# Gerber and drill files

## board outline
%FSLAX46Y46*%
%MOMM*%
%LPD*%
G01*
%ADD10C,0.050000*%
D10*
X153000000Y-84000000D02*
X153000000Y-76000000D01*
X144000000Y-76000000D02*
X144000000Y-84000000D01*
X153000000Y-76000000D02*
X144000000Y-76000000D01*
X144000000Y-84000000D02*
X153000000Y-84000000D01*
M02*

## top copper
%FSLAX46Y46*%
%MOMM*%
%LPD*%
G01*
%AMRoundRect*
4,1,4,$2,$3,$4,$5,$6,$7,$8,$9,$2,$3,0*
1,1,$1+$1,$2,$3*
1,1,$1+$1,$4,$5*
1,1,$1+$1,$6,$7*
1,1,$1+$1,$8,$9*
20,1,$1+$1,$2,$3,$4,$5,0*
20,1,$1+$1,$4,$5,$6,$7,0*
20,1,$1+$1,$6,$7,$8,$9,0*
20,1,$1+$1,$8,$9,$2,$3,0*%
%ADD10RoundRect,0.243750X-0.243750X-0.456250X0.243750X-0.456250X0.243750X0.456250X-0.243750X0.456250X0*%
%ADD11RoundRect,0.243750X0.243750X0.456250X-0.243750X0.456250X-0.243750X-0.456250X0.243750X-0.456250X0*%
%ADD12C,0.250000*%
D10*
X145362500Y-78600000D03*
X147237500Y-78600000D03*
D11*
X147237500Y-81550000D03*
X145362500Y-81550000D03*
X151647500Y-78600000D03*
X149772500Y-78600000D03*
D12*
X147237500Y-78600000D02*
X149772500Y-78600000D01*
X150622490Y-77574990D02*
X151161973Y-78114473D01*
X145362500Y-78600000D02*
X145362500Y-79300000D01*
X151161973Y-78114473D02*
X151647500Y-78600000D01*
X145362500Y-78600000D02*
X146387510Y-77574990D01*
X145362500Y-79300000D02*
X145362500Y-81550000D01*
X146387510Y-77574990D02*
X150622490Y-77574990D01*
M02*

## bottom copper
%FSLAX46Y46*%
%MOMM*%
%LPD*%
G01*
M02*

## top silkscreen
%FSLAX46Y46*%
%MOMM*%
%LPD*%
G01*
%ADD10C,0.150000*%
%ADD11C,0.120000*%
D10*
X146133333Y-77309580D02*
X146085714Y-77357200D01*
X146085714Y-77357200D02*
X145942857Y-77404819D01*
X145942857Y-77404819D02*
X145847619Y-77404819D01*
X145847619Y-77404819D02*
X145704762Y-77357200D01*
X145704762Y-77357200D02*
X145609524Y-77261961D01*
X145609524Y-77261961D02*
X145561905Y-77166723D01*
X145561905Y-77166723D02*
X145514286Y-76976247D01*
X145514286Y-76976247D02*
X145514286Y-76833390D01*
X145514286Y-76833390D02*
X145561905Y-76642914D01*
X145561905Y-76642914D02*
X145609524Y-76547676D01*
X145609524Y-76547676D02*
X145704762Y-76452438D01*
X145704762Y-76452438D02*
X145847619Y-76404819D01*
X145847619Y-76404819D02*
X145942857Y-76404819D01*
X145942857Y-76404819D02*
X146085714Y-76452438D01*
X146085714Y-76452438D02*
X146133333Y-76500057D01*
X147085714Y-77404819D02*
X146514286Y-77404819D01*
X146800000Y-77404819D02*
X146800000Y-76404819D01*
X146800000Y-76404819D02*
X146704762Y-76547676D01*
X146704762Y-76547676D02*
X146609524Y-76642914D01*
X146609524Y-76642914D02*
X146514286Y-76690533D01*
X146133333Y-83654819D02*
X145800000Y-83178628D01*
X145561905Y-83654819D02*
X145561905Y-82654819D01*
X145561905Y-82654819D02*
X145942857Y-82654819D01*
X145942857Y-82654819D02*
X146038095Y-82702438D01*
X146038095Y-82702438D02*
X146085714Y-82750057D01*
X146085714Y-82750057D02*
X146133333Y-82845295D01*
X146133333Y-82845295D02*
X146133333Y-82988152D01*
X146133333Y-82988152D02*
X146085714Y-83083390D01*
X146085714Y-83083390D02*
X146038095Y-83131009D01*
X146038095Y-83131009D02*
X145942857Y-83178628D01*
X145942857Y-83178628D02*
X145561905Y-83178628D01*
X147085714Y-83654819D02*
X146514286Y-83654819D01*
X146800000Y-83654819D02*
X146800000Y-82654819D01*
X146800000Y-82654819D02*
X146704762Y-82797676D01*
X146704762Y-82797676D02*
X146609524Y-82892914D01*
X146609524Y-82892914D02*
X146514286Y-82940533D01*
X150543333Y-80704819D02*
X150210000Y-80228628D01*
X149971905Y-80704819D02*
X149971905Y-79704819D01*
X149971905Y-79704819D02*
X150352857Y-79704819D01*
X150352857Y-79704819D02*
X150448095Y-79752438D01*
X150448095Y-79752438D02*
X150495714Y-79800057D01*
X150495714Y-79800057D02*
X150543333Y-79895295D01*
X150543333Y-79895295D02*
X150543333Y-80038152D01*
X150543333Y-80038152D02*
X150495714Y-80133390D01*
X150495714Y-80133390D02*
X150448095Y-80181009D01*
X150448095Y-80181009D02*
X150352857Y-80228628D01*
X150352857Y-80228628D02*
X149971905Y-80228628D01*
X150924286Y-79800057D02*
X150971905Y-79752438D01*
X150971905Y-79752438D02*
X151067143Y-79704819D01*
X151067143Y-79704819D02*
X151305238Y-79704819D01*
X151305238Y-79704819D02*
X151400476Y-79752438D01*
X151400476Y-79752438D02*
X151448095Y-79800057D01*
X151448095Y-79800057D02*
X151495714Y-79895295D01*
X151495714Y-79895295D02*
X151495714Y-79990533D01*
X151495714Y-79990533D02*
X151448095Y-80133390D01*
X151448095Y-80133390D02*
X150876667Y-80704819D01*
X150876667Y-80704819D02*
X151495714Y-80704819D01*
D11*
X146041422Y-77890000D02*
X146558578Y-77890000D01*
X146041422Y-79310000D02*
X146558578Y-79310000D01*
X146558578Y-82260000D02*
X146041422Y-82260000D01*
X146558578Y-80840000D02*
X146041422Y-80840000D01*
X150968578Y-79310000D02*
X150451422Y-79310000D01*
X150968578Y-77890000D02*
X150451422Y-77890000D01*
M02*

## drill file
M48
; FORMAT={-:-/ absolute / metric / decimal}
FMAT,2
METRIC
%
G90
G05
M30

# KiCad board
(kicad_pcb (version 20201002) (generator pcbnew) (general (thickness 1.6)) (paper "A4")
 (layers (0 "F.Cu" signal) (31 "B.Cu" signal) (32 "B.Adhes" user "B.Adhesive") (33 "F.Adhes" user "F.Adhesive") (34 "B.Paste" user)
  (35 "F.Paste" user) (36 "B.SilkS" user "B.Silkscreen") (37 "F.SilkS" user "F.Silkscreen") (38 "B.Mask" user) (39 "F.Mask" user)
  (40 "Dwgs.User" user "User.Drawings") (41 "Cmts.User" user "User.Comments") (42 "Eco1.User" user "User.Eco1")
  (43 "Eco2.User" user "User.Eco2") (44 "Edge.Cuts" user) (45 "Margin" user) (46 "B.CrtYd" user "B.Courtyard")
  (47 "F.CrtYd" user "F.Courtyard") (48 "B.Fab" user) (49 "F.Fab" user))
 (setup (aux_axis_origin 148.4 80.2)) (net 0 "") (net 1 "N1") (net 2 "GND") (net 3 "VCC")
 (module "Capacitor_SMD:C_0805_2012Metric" (layer "F.Cu") (at 146.3 78.6)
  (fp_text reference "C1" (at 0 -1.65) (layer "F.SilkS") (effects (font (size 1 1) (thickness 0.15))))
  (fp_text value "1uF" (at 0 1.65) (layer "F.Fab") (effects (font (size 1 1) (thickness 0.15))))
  (fp_line (start -0.258578 -0.71) (end 0.258578 -0.71) (layer "F.SilkS") (width 0.12))
  (fp_line (start -0.258578 0.71) (end 0.258578 0.71) (layer "F.SilkS") (width 0.12))
  (pad "1" smd roundrect (at -0.9375 0) (size 0.975 1.4) (layers "F.Cu" "F.Paste" "F.Mask") (roundrect_rratio 0.25) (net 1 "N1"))
  (pad "2" smd roundrect (at 0.9375 0) (size 0.975 1.4) (layers "F.Cu" "F.Paste" "F.Mask") (roundrect_rratio 0.25) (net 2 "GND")))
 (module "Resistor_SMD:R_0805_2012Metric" (layer "F.Cu") (at 146.3 81.55 180)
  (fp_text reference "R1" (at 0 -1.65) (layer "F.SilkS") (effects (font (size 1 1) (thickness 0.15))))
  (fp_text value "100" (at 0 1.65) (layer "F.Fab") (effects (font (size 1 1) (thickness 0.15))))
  (fp_line (start -0.258578 -0.71) (end 0.258578 -0.71) (layer "F.SilkS") (width 0.12))
  (fp_line (start -0.258578 0.71) (end 0.258578 0.71) (layer "F.SilkS") (width 0.12))
  (pad "1" smd roundrect (at -0.9375 0 180) (size 0.975 1.4) (layers "F.Cu" "F.Paste" "F.Mask") (roundrect_rratio 0.25) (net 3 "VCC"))
  (pad "2" smd roundrect (at 0.9375 0 180) (size 0.975 1.4) (layers "F.Cu" "F.Paste" "F.Mask") (roundrect_rratio 0.25) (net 1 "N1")))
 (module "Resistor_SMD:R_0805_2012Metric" (layer "F.Cu") (at 150.71 78.6 180)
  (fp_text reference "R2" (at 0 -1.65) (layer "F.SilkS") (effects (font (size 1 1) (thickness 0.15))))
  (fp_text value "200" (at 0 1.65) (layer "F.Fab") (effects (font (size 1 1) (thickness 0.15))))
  (fp_line (start -0.258578 -0.71) (end 0.258578 -0.71) (layer "F.SilkS") (width 0.12))
  (fp_line (start -0.258578 0.71) (end 0.258578 0.71) (layer "F.SilkS") (width 0.12))
  (pad "1" smd roundrect (at -0.9375 0 180) (size 0.975 1.4) (layers "F.Cu" "F.Paste" "F.Mask") (roundrect_rratio 0.25) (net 1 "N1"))
  (pad "2" smd roundrect (at 0.9375 0 180) (size 0.975 1.4) (layers "F.Cu" "F.Paste" "F.Mask") (roundrect_rratio 0.25) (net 2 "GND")))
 (gr_line (start 153 84) (end 153 76) (layer "Edge.Cuts") (width 0.05))
 (gr_line (start 144 76) (end 144 84) (layer "Edge.Cuts") (width 0.05))
 (gr_line (start 153 76) (end 144 76) (layer "Edge.Cuts") (width 0.05))
 (gr_line (start 144 84) (end 153 84) (layer "Edge.Cuts") (width 0.05))
 (segment (start 147.2375 78.6) (end 149.7725 78.6) (width 0.25) (layer "F.Cu") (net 2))
 (segment (start 150.62249 77.57499) (end 151.161973 78.114473) (width 0.25) (layer "F.Cu") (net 1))
 (segment (start 145.3625 78.6) (end 145.3625 79.3) (width 0.25) (layer "F.Cu") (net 1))
 (segment (start 151.161973 78.114473) (end 151.6475 78.6) (width 0.25) (layer "F.Cu") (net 1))
 (segment (start 145.3625 78.6) (end 146.38751 77.57499) (width 0.25) (layer "F.Cu") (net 1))
 (segment (start 145.3625 79.3) (end 145.3625 81.55) (width 0.25) (layer "F.Cu") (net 1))
 (segment (start 146.38751 77.57499) (end 150.62249 77.57499) (width 0.25) (layer "F.Cu") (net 1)))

